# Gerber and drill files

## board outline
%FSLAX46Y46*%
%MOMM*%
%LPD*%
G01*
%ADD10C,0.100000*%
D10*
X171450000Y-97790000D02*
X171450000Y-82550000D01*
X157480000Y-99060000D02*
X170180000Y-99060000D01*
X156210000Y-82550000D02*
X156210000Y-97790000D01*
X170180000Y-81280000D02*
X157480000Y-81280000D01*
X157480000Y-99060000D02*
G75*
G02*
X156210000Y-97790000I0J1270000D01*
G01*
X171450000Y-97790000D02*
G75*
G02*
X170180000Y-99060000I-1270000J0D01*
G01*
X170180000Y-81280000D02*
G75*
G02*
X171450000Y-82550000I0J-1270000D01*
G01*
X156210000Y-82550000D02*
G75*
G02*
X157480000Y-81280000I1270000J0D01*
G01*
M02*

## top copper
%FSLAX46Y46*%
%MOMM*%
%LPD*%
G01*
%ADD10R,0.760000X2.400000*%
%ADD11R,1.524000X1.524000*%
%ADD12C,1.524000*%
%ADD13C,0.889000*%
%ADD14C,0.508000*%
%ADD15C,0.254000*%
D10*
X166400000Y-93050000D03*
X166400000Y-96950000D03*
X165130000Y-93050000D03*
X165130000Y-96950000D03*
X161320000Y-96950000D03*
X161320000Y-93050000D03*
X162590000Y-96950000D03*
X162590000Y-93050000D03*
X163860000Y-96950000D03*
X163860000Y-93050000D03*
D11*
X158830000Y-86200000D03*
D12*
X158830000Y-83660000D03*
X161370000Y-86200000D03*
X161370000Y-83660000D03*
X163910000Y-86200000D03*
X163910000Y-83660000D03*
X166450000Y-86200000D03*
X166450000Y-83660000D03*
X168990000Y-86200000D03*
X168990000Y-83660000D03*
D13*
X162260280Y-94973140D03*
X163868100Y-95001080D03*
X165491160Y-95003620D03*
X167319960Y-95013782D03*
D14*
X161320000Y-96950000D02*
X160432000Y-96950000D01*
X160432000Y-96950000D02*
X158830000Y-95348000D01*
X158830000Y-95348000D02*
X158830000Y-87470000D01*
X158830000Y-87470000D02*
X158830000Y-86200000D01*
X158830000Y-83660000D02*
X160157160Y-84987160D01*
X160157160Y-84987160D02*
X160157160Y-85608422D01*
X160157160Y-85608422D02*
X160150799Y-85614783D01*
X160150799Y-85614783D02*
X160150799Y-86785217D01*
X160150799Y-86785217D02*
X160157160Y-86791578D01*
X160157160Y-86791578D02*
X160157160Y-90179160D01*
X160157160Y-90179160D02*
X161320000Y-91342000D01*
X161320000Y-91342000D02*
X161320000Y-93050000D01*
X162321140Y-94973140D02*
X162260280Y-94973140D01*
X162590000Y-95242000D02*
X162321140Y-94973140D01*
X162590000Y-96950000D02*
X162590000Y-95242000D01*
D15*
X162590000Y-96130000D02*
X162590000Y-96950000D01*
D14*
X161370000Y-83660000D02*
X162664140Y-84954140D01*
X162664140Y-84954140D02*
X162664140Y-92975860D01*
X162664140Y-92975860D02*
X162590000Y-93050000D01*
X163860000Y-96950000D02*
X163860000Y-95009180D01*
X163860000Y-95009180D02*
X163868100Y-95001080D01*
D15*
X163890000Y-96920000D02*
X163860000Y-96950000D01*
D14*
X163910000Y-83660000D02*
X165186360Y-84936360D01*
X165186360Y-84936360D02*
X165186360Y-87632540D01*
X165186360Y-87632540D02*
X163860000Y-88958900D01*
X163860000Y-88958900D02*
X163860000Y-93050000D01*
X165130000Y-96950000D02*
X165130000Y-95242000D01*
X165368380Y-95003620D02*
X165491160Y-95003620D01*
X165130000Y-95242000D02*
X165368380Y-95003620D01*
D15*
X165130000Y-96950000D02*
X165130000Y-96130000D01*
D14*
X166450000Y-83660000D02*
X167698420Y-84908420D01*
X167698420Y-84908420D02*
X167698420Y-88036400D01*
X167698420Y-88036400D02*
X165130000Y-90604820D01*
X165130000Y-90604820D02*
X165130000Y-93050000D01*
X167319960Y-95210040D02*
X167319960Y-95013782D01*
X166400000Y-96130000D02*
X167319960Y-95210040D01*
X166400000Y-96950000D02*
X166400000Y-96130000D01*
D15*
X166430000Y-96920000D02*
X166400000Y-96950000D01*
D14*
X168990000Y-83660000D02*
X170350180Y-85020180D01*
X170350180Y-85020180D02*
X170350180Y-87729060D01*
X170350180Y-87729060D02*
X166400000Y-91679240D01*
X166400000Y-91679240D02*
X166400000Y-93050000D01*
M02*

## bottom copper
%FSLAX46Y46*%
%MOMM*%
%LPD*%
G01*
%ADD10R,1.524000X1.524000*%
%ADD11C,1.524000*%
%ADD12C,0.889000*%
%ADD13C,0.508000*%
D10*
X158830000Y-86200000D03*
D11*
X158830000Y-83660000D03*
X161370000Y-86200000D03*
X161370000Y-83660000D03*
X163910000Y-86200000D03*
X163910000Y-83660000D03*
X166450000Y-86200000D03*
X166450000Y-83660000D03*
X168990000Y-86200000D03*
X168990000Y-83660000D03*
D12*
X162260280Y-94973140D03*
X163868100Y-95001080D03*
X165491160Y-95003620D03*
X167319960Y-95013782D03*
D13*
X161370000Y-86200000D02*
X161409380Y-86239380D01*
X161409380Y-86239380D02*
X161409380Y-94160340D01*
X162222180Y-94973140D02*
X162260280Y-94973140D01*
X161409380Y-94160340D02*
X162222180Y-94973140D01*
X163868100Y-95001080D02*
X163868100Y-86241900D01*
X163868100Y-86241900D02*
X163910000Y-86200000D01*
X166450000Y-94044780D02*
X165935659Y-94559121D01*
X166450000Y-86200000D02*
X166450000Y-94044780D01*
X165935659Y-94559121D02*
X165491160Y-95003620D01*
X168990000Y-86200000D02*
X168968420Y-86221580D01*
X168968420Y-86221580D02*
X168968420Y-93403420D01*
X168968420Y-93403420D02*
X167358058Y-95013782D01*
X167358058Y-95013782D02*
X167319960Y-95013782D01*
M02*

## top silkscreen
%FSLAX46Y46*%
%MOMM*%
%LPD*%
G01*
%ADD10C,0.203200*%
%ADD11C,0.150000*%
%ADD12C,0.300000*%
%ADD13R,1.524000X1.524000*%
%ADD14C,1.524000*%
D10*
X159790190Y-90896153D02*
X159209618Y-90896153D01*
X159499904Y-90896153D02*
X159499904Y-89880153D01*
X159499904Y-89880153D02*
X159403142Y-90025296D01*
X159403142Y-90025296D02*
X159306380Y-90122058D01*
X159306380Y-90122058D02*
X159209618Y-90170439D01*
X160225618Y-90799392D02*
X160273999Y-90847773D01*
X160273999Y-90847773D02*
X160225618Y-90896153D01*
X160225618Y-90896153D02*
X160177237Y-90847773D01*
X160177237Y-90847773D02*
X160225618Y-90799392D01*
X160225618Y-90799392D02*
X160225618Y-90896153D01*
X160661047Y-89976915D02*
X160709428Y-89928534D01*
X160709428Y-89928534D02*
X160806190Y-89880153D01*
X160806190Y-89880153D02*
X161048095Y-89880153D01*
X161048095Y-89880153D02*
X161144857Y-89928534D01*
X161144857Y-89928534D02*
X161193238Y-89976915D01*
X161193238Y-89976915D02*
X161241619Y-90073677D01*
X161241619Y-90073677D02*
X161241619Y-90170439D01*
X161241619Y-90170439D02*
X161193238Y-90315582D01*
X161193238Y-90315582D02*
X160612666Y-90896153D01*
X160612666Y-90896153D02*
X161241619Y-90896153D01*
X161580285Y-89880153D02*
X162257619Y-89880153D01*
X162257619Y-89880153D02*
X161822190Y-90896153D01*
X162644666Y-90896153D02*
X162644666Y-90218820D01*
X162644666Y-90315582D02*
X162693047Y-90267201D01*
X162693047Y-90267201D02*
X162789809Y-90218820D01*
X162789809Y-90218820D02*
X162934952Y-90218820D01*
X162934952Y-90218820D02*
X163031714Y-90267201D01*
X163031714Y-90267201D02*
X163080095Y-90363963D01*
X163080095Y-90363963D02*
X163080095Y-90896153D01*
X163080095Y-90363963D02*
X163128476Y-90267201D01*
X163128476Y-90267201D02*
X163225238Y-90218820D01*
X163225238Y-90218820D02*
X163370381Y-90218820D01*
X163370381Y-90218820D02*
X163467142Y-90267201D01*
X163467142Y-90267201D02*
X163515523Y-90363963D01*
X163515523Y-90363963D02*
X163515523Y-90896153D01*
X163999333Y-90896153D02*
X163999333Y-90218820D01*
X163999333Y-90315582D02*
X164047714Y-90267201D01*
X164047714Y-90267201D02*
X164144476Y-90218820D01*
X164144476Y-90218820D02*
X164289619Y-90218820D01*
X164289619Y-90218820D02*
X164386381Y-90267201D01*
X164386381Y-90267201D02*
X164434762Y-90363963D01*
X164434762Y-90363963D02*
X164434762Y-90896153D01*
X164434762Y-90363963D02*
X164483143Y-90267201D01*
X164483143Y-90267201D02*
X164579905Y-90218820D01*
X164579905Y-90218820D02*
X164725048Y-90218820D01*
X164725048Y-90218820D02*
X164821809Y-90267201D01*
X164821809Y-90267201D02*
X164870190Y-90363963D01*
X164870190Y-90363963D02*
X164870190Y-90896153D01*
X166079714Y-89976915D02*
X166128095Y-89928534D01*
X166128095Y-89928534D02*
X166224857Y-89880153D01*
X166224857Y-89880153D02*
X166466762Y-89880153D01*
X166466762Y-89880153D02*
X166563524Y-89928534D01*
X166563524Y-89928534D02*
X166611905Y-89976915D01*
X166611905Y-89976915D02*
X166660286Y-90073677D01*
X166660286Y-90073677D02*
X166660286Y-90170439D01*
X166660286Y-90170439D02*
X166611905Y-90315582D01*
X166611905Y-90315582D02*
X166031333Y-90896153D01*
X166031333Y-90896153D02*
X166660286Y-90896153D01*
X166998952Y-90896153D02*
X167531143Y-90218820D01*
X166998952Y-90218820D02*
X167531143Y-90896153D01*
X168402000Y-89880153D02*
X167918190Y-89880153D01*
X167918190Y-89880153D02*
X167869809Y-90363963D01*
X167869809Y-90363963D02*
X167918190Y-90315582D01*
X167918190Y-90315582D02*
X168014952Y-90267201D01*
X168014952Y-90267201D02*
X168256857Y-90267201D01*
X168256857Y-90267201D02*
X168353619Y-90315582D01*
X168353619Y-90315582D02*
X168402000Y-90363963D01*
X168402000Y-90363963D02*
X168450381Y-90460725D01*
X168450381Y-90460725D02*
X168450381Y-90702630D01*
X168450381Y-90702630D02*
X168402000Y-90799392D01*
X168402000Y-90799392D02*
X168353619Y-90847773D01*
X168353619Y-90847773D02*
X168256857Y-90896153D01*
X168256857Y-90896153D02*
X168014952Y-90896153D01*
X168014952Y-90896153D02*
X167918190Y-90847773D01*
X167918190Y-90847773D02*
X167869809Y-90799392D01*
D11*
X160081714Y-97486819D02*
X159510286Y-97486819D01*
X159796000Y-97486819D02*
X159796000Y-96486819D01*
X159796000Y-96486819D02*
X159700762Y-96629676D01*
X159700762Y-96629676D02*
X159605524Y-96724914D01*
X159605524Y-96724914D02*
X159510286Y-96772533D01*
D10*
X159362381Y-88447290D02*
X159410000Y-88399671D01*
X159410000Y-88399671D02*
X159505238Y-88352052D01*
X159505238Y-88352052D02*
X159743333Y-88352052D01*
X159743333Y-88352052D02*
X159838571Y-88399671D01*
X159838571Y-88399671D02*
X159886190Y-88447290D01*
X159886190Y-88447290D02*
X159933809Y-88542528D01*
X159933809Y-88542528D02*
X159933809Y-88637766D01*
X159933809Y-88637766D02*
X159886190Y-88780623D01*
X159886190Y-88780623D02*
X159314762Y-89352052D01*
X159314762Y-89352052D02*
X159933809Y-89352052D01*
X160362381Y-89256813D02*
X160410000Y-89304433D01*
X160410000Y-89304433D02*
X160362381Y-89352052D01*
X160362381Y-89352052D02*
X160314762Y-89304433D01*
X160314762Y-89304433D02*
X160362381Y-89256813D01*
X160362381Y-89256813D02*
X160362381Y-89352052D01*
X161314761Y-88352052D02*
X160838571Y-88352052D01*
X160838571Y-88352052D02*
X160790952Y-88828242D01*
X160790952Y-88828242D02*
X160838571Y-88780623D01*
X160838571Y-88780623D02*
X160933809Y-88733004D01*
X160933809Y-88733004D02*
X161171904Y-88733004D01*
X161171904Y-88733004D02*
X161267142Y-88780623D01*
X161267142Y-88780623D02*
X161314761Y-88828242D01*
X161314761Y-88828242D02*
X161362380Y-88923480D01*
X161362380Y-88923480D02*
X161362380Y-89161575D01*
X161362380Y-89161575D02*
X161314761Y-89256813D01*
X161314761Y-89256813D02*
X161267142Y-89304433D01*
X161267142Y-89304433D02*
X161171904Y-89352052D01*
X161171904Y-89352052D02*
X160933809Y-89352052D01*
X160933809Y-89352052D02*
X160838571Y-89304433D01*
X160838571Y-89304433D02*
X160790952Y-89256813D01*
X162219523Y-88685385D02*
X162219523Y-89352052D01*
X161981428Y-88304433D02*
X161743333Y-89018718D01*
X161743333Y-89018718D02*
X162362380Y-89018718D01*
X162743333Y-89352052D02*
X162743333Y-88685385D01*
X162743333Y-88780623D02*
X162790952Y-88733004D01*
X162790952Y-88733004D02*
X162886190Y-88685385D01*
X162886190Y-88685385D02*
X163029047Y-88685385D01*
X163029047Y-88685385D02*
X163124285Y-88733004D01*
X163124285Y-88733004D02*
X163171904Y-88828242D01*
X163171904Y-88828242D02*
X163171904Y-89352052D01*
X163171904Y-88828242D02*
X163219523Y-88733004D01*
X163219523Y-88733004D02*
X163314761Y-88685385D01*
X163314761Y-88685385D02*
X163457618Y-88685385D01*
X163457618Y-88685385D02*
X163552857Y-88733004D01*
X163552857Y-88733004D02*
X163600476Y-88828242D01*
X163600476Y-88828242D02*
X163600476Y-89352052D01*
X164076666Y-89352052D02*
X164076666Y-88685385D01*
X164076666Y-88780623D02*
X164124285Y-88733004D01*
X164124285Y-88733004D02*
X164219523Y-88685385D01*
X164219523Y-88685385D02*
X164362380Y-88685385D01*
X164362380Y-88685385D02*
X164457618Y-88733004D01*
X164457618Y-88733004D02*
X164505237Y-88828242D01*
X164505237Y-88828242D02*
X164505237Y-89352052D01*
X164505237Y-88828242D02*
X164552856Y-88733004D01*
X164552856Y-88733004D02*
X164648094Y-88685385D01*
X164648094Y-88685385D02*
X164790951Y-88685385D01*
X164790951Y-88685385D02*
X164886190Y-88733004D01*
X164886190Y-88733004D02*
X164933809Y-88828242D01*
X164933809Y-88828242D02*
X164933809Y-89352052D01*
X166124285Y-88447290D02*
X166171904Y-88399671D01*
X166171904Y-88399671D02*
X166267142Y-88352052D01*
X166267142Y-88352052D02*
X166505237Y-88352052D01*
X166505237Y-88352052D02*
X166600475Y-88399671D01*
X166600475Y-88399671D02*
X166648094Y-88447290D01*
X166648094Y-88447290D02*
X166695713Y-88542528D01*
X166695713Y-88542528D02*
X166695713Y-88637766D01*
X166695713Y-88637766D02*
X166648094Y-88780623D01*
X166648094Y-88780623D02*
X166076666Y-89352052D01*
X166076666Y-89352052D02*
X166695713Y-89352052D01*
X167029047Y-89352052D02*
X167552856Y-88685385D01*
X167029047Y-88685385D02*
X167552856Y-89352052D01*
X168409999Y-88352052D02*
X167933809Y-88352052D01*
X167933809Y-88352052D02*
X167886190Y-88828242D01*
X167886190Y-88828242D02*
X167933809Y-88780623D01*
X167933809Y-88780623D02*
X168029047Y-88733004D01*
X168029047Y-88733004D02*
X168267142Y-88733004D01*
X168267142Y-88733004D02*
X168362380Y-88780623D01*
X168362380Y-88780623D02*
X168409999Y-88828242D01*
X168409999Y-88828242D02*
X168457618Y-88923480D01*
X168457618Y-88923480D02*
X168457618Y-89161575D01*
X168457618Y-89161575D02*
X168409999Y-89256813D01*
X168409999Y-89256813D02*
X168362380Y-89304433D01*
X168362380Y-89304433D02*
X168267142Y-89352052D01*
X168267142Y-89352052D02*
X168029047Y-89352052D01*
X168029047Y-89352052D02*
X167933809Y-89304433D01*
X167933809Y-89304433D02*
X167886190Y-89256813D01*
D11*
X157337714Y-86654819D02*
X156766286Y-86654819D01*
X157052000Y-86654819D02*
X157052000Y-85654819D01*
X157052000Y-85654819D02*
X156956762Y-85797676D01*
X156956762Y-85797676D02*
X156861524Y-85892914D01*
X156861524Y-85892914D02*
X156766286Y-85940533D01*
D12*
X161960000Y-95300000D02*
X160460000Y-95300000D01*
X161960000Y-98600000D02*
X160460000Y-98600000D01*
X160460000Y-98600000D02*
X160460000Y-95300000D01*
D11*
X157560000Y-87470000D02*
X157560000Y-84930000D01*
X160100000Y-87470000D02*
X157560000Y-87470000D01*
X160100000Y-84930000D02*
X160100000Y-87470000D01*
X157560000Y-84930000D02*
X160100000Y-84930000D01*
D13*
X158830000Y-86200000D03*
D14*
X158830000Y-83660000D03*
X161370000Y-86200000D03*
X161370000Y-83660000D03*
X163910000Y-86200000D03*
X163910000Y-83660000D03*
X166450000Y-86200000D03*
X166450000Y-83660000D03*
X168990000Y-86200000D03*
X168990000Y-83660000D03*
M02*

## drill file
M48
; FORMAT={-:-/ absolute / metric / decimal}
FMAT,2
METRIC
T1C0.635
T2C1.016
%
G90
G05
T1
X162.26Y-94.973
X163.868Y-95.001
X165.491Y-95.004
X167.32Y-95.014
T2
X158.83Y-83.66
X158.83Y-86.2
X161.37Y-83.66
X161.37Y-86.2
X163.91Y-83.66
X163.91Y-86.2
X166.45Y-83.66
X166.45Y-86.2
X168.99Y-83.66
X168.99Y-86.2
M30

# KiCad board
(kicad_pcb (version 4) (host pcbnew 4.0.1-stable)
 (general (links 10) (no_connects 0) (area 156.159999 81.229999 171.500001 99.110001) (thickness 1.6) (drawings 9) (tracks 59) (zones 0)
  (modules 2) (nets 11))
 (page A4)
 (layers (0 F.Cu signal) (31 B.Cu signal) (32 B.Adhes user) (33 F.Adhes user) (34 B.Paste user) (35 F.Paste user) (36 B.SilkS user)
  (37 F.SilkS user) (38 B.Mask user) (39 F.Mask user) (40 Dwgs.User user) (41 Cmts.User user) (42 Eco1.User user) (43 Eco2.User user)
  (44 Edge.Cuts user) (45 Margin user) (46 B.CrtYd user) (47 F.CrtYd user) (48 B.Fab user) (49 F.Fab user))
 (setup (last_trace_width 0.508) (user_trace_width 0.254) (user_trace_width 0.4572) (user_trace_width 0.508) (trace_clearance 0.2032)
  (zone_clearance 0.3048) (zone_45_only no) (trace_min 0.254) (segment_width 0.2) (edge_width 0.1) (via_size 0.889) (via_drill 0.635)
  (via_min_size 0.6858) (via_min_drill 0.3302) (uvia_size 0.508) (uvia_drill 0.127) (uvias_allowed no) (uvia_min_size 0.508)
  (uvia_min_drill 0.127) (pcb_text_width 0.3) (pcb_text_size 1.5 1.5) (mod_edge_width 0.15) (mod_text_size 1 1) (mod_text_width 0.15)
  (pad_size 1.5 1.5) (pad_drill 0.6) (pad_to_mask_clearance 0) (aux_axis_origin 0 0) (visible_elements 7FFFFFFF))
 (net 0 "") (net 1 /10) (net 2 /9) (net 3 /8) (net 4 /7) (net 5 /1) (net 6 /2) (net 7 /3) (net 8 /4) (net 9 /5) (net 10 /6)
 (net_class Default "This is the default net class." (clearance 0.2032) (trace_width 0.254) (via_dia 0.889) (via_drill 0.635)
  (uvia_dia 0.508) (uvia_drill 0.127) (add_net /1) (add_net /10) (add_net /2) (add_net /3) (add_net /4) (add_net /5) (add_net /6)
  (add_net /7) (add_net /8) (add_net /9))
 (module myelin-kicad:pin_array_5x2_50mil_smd (layer F.Cu) (at 163.86 95)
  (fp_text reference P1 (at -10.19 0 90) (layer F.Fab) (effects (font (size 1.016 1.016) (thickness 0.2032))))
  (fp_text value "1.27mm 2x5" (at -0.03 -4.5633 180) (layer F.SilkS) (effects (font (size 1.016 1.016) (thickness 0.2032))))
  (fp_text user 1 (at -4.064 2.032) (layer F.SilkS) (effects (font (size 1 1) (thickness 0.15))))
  (fp_line (start -1.9 0.3) (end -3.4 0.3) (layer F.SilkS) (width 0.3))
  (fp_line (start -1.9 3.6) (end -3.4 3.6) (layer F.SilkS) (width 0.3))
  (fp_line (start -3.4 3.6) (end -3.4 0.3) (layer F.SilkS) (width 0.3))
  (pad 10 smd rect (at 2.54 -1.95) (size 0.76 2.4) (layers F.Cu F.Paste F.Mask) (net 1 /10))
  (pad 9 smd rect (at 2.54 1.95) (size 0.76 2.4) (layers F.Cu F.Paste F.Mask) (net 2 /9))
  (pad 8 smd rect (at 1.27 -1.95) (size 0.76 2.4) (layers F.Cu F.Paste F.Mask) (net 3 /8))
  (pad 7 smd rect (at 1.27 1.95) (size 0.76 2.4) (layers F.Cu F.Paste F.Mask) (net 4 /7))
  (pad 1 smd rect (at -2.54 1.95) (size 0.76 2.4) (layers F.Cu F.Paste F.Mask) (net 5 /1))
  (pad 2 smd rect (at -2.54 -1.95) (size 0.76 2.4) (layers F.Cu F.Paste F.Mask) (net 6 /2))
  (pad 3 smd rect (at -1.27 1.95) (size 0.76 2.4) (layers F.Cu F.Paste F.Mask) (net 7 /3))
  (pad 4 smd rect (at -1.27 -1.95) (size 0.76 2.4) (layers F.Cu F.Paste F.Mask) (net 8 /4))
  (pad 5 smd rect (at 0 1.95) (size 0.76 2.4) (layers F.Cu F.Paste F.Mask) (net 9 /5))
  (pad 6 smd rect (at 0 -1.95) (size 0.76 2.4) (layers F.Cu F.Paste F.Mask) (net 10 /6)))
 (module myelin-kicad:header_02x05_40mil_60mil (layer F.Cu) (at 163.91 84.93)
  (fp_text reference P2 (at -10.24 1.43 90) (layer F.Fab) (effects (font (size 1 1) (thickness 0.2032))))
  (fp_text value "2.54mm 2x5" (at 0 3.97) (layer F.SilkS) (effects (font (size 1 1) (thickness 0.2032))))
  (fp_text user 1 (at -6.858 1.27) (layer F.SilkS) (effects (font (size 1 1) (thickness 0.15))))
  (fp_line (start -6.35 2.54) (end -6.35 0) (layer F.SilkS) (width 0.15))
  (fp_line (start -3.81 2.54) (end -6.35 2.54) (layer F.SilkS) (width 0.15))
  (fp_line (start -3.81 0) (end -3.81 2.54) (layer F.SilkS) (width 0.15))
  (fp_line (start -6.35 0) (end -3.81 0) (layer F.SilkS) (width 0.15))
  (pad 1 thru_hole rect (at -5.08 1.27) (size 1.524 1.524) (drill 1.016) (layers *.Cu *.Mask F.SilkS) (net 5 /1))
  (pad 2 thru_hole circle (at -5.08 -1.27) (size 1.524 1.524) (drill 1.016) (layers *.Cu *.Mask F.SilkS) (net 6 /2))
  (pad 3 thru_hole circle (at -2.54 1.27) (size 1.524 1.524) (drill 1.016) (layers *.Cu *.Mask F.SilkS) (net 7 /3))
  (pad 4 thru_hole circle (at -2.54 -1.27) (size 1.524 1.524) (drill 1.016) (layers *.Cu *.Mask F.SilkS) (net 8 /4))
  (pad 5 thru_hole circle (at 0 1.27) (size 1.524 1.524) (drill 1.016) (layers *.Cu *.Mask F.SilkS) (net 9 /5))
  (pad 6 thru_hole circle (at 0 -1.27) (size 1.524 1.524) (drill 1.016) (layers *.Cu *.Mask F.SilkS) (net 10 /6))
  (pad 7 thru_hole circle (at 2.54 1.27) (size 1.524 1.524) (drill 1.016) (layers *.Cu *.Mask F.SilkS) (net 4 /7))
  (pad 8 thru_hole circle (at 2.54 -1.27) (size 1.524 1.524) (drill 1.016) (layers *.Cu *.Mask F.SilkS) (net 3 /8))
  (pad 9 thru_hole circle (at 5.08 1.27) (size 1.524 1.524) (drill 1.016) (layers *.Cu *.Mask F.SilkS) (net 2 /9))
  (pad 10 thru_hole circle (at 5.08 -1.27) (size 1.524 1.524) (drill 1.016) (layers *.Cu *.Mask F.SilkS) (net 1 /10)))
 (gr_line (start 171.45 97.79) (end 171.45 82.55) (layer Edge.Cuts) (width 0.1))
 (gr_line (start 157.48 99.06) (end 170.18 99.06) (layer Edge.Cuts) (width 0.1))
 (gr_line (start 156.21 82.55) (end 156.21 97.79) (layer Edge.Cuts) (width 0.1))
 (gr_line (start 170.18 81.28) (end 157.48 81.28) (layer Edge.Cuts) (width 0.1))
 (gr_arc (start 157.48 97.79) (end 157.48 99.06) (angle 90) (layer Edge.Cuts) (width 0.1))
 (gr_arc (start 170.18 97.79) (end 171.45 97.79) (angle 90) (layer Edge.Cuts) (width 0.1))
 (gr_arc (start 170.18 82.55) (end 170.18 81.28) (angle 90) (layer Edge.Cuts) (width 0.1))
 (gr_arc (start 157.48 82.55) (end 156.21 82.55) (angle 90) (layer Edge.Cuts) (width 0.1))
 (segment (start 161.32 96.95) (end 160.432 96.95) (width 0.508) (layer F.Cu) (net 5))
 (segment (start 160.432 96.95) (end 158.83 95.348) (width 0.508) (layer F.Cu) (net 5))
 (segment (start 158.83 95.348) (end 158.83 87.47) (width 0.508) (layer F.Cu) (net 5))
 (segment (start 158.83 87.47) (end 158.83 86.2) (width 0.508) (layer F.Cu) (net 5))
 (segment (start 158.83 83.66) (end 160.15716 84.98716) (width 0.508) (layer F.Cu) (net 6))
 (segment (start 160.15716 84.98716) (end 160.15716 85.608422) (width 0.508) (layer F.Cu) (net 6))
 (segment (start 160.15716 85.608422) (end 160.150799 85.614783) (width 0.508) (layer F.Cu) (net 6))
 (segment (start 160.150799 85.614783) (end 160.150799 86.785217) (width 0.508) (layer F.Cu) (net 6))
 (segment (start 160.150799 86.785217) (end 160.15716 86.791578) (width 0.508) (layer F.Cu) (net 6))
 (segment (start 160.15716 86.791578) (end 160.15716 90.17916) (width 0.508) (layer F.Cu) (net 6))
 (segment (start 160.15716 90.17916) (end 161.32 91.342) (width 0.508) (layer F.Cu) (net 6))
 (segment (start 161.32 91.342) (end 161.32 93.05) (width 0.508) (layer F.Cu) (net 6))
 (segment (start 161.37 86.2) (end 161.40938 86.23938) (width 0.508) (layer B.Cu) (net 7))
 (segment (start 161.40938 86.23938) (end 161.40938 94.16034) (width 0.508) (layer B.Cu) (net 7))
 (segment (start 162.22218 94.97314) (end 162.26028 94.97314) (width 0.508) (layer B.Cu) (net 7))
 (segment (start 161.40938 94.16034) (end 162.22218 94.97314) (width 0.508) (layer B.Cu) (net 7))
 (segment (start 162.32114 94.97314) (end 162.26028 94.97314) (width 0.508) (layer F.Cu) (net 7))
 (segment (start 162.59 95.242) (end 162.32114 94.97314) (width 0.508) (layer F.Cu) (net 7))
 (segment (start 162.59 96.95) (end 162.59 95.242) (width 0.508) (layer F.Cu) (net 7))
 (via (at 162.26028 94.97314) (size 0.889) (drill 0.635) (layers F.Cu B.Cu) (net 7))
 (segment (start 162.59 96.13) (end 162.59 96.95) (width 0.254) (layer F.Cu) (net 7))
 (segment (start 161.37 83.66) (end 162.66414 84.95414) (width 0.508) (layer F.Cu) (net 8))
 (segment (start 162.66414 84.95414) (end 162.66414 92.97586) (width 0.508) (layer F.Cu) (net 8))
 (segment (start 162.66414 92.97586) (end 162.59 93.05) (width 0.508) (layer F.Cu) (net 8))
 (segment (start 163.8681 95.00108) (end 163.8681 86.2419) (width 0.508) (layer B.Cu) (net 9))
 (segment (start 163.8681 86.2419) (end 163.91 86.2) (width 0.508) (layer B.Cu) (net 9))
 (segment (start 163.86 96.95) (end 163.86 95.00918) (width 0.508) (layer F.Cu) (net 9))
 (segment (start 163.86 95.00918) (end 163.8681 95.00108) (width 0.508) (layer F.Cu) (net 9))
 (via (at 163.8681 95.00108) (size 0.889) (drill 0.635) (layers F.Cu B.Cu) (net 9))
 (segment (start 163.89 96.92) (end 163.86 96.95) (width 0.254) (layer F.Cu) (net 9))
 (segment (start 163.91 83.66) (end 165.18636 84.93636) (width 0.508) (layer F.Cu) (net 10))
 (segment (start 165.18636 84.93636) (end 165.18636 87.63254) (width 0.508) (layer F.Cu) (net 10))
 (segment (start 165.18636 87.63254) (end 163.86 88.9589) (width 0.508) (layer F.Cu) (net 10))
 (segment (start 163.86 88.9589) (end 163.86 93.05) (width 0.508) (layer F.Cu) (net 10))
 (segment (start 165.13 96.95) (end 165.13 95.242) (width 0.508) (layer F.Cu) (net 4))
 (segment (start 166.45 94.04478) (end 165.935659 94.559121) (width 0.508) (layer B.Cu) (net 4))
 (segment (start 165.36838 95.00362) (end 165.49116 95.00362) (width 0.508) (layer F.Cu) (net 4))
 (segment (start 166.45 86.2) (end 166.45 94.04478) (width 0.508) (layer B.Cu) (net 4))
 (segment (start 165.13 95.242) (end 165.36838 95.00362) (width 0.508) (layer F.Cu) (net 4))
 (segment (start 165.935659 94.559121) (end 165.49116 95.00362) (width 0.508) (layer B.Cu) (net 4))
 (via (at 165.49116 95.00362) (size 0.889) (drill 0.635) (layers F.Cu B.Cu) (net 4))
 (segment (start 165.13 96.95) (end 165.13 96.13) (width 0.254) (layer F.Cu) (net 4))
 (segment (start 166.45 83.66) (end 167.69842 84.90842) (width 0.508) (layer F.Cu) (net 3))
 (segment (start 167.69842 84.90842) (end 167.69842 88.0364) (width 0.508) (layer F.Cu) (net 3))
 (segment (start 167.69842 88.0364) (end 165.13 90.60482) (width 0.508) (layer F.Cu) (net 3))
 (segment (start 165.13 90.60482) (end 165.13 93.05) (width 0.508) (layer F.Cu) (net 3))
 (segment (start 168.99 86.2) (end 168.96842 86.22158) (width 0.508) (layer B.Cu) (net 2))
 (segment (start 168.96842 86.22158) (end 168.96842 93.40342) (width 0.508) (layer B.Cu) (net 2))
 (segment (start 168.96842 93.40342) (end 167.358058 95.013782) (width 0.508) (layer B.Cu) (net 2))
 (segment (start 167.358058 95.013782) (end 167.31996 95.013782) (width 0.508) (layer B.Cu) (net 2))
 (segment (start 167.31996 95.21004) (end 167.31996 95.013782) (width 0.508) (layer F.Cu) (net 2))
 (segment (start 166.4 96.13) (end 167.31996 95.21004) (width 0.508) (layer F.Cu) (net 2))
 (segment (start 166.4 96.95) (end 166.4 96.13) (width 0.508) (layer F.Cu) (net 2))
 (via (at 167.31996 95.013782) (size 0.889) (drill 0.635) (layers F.Cu B.Cu) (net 2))
 (segment (start 166.43 96.92) (end 166.4 96.95) (width 0.254) (layer F.Cu) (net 2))
 (segment (start 168.99 83.66) (end 170.35018 85.02018) (width 0.508) (layer F.Cu) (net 1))
 (segment (start 170.35018 85.02018) (end 170.35018 87.72906) (width 0.508) (layer F.Cu) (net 1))
 (segment (start 170.35018 87.72906) (end 166.4 91.67924) (width 0.508) (layer F.Cu) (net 1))
 (segment (start 166.4 91.67924) (end 166.4 93.05) (width 0.508) (layer F.Cu) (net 1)))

